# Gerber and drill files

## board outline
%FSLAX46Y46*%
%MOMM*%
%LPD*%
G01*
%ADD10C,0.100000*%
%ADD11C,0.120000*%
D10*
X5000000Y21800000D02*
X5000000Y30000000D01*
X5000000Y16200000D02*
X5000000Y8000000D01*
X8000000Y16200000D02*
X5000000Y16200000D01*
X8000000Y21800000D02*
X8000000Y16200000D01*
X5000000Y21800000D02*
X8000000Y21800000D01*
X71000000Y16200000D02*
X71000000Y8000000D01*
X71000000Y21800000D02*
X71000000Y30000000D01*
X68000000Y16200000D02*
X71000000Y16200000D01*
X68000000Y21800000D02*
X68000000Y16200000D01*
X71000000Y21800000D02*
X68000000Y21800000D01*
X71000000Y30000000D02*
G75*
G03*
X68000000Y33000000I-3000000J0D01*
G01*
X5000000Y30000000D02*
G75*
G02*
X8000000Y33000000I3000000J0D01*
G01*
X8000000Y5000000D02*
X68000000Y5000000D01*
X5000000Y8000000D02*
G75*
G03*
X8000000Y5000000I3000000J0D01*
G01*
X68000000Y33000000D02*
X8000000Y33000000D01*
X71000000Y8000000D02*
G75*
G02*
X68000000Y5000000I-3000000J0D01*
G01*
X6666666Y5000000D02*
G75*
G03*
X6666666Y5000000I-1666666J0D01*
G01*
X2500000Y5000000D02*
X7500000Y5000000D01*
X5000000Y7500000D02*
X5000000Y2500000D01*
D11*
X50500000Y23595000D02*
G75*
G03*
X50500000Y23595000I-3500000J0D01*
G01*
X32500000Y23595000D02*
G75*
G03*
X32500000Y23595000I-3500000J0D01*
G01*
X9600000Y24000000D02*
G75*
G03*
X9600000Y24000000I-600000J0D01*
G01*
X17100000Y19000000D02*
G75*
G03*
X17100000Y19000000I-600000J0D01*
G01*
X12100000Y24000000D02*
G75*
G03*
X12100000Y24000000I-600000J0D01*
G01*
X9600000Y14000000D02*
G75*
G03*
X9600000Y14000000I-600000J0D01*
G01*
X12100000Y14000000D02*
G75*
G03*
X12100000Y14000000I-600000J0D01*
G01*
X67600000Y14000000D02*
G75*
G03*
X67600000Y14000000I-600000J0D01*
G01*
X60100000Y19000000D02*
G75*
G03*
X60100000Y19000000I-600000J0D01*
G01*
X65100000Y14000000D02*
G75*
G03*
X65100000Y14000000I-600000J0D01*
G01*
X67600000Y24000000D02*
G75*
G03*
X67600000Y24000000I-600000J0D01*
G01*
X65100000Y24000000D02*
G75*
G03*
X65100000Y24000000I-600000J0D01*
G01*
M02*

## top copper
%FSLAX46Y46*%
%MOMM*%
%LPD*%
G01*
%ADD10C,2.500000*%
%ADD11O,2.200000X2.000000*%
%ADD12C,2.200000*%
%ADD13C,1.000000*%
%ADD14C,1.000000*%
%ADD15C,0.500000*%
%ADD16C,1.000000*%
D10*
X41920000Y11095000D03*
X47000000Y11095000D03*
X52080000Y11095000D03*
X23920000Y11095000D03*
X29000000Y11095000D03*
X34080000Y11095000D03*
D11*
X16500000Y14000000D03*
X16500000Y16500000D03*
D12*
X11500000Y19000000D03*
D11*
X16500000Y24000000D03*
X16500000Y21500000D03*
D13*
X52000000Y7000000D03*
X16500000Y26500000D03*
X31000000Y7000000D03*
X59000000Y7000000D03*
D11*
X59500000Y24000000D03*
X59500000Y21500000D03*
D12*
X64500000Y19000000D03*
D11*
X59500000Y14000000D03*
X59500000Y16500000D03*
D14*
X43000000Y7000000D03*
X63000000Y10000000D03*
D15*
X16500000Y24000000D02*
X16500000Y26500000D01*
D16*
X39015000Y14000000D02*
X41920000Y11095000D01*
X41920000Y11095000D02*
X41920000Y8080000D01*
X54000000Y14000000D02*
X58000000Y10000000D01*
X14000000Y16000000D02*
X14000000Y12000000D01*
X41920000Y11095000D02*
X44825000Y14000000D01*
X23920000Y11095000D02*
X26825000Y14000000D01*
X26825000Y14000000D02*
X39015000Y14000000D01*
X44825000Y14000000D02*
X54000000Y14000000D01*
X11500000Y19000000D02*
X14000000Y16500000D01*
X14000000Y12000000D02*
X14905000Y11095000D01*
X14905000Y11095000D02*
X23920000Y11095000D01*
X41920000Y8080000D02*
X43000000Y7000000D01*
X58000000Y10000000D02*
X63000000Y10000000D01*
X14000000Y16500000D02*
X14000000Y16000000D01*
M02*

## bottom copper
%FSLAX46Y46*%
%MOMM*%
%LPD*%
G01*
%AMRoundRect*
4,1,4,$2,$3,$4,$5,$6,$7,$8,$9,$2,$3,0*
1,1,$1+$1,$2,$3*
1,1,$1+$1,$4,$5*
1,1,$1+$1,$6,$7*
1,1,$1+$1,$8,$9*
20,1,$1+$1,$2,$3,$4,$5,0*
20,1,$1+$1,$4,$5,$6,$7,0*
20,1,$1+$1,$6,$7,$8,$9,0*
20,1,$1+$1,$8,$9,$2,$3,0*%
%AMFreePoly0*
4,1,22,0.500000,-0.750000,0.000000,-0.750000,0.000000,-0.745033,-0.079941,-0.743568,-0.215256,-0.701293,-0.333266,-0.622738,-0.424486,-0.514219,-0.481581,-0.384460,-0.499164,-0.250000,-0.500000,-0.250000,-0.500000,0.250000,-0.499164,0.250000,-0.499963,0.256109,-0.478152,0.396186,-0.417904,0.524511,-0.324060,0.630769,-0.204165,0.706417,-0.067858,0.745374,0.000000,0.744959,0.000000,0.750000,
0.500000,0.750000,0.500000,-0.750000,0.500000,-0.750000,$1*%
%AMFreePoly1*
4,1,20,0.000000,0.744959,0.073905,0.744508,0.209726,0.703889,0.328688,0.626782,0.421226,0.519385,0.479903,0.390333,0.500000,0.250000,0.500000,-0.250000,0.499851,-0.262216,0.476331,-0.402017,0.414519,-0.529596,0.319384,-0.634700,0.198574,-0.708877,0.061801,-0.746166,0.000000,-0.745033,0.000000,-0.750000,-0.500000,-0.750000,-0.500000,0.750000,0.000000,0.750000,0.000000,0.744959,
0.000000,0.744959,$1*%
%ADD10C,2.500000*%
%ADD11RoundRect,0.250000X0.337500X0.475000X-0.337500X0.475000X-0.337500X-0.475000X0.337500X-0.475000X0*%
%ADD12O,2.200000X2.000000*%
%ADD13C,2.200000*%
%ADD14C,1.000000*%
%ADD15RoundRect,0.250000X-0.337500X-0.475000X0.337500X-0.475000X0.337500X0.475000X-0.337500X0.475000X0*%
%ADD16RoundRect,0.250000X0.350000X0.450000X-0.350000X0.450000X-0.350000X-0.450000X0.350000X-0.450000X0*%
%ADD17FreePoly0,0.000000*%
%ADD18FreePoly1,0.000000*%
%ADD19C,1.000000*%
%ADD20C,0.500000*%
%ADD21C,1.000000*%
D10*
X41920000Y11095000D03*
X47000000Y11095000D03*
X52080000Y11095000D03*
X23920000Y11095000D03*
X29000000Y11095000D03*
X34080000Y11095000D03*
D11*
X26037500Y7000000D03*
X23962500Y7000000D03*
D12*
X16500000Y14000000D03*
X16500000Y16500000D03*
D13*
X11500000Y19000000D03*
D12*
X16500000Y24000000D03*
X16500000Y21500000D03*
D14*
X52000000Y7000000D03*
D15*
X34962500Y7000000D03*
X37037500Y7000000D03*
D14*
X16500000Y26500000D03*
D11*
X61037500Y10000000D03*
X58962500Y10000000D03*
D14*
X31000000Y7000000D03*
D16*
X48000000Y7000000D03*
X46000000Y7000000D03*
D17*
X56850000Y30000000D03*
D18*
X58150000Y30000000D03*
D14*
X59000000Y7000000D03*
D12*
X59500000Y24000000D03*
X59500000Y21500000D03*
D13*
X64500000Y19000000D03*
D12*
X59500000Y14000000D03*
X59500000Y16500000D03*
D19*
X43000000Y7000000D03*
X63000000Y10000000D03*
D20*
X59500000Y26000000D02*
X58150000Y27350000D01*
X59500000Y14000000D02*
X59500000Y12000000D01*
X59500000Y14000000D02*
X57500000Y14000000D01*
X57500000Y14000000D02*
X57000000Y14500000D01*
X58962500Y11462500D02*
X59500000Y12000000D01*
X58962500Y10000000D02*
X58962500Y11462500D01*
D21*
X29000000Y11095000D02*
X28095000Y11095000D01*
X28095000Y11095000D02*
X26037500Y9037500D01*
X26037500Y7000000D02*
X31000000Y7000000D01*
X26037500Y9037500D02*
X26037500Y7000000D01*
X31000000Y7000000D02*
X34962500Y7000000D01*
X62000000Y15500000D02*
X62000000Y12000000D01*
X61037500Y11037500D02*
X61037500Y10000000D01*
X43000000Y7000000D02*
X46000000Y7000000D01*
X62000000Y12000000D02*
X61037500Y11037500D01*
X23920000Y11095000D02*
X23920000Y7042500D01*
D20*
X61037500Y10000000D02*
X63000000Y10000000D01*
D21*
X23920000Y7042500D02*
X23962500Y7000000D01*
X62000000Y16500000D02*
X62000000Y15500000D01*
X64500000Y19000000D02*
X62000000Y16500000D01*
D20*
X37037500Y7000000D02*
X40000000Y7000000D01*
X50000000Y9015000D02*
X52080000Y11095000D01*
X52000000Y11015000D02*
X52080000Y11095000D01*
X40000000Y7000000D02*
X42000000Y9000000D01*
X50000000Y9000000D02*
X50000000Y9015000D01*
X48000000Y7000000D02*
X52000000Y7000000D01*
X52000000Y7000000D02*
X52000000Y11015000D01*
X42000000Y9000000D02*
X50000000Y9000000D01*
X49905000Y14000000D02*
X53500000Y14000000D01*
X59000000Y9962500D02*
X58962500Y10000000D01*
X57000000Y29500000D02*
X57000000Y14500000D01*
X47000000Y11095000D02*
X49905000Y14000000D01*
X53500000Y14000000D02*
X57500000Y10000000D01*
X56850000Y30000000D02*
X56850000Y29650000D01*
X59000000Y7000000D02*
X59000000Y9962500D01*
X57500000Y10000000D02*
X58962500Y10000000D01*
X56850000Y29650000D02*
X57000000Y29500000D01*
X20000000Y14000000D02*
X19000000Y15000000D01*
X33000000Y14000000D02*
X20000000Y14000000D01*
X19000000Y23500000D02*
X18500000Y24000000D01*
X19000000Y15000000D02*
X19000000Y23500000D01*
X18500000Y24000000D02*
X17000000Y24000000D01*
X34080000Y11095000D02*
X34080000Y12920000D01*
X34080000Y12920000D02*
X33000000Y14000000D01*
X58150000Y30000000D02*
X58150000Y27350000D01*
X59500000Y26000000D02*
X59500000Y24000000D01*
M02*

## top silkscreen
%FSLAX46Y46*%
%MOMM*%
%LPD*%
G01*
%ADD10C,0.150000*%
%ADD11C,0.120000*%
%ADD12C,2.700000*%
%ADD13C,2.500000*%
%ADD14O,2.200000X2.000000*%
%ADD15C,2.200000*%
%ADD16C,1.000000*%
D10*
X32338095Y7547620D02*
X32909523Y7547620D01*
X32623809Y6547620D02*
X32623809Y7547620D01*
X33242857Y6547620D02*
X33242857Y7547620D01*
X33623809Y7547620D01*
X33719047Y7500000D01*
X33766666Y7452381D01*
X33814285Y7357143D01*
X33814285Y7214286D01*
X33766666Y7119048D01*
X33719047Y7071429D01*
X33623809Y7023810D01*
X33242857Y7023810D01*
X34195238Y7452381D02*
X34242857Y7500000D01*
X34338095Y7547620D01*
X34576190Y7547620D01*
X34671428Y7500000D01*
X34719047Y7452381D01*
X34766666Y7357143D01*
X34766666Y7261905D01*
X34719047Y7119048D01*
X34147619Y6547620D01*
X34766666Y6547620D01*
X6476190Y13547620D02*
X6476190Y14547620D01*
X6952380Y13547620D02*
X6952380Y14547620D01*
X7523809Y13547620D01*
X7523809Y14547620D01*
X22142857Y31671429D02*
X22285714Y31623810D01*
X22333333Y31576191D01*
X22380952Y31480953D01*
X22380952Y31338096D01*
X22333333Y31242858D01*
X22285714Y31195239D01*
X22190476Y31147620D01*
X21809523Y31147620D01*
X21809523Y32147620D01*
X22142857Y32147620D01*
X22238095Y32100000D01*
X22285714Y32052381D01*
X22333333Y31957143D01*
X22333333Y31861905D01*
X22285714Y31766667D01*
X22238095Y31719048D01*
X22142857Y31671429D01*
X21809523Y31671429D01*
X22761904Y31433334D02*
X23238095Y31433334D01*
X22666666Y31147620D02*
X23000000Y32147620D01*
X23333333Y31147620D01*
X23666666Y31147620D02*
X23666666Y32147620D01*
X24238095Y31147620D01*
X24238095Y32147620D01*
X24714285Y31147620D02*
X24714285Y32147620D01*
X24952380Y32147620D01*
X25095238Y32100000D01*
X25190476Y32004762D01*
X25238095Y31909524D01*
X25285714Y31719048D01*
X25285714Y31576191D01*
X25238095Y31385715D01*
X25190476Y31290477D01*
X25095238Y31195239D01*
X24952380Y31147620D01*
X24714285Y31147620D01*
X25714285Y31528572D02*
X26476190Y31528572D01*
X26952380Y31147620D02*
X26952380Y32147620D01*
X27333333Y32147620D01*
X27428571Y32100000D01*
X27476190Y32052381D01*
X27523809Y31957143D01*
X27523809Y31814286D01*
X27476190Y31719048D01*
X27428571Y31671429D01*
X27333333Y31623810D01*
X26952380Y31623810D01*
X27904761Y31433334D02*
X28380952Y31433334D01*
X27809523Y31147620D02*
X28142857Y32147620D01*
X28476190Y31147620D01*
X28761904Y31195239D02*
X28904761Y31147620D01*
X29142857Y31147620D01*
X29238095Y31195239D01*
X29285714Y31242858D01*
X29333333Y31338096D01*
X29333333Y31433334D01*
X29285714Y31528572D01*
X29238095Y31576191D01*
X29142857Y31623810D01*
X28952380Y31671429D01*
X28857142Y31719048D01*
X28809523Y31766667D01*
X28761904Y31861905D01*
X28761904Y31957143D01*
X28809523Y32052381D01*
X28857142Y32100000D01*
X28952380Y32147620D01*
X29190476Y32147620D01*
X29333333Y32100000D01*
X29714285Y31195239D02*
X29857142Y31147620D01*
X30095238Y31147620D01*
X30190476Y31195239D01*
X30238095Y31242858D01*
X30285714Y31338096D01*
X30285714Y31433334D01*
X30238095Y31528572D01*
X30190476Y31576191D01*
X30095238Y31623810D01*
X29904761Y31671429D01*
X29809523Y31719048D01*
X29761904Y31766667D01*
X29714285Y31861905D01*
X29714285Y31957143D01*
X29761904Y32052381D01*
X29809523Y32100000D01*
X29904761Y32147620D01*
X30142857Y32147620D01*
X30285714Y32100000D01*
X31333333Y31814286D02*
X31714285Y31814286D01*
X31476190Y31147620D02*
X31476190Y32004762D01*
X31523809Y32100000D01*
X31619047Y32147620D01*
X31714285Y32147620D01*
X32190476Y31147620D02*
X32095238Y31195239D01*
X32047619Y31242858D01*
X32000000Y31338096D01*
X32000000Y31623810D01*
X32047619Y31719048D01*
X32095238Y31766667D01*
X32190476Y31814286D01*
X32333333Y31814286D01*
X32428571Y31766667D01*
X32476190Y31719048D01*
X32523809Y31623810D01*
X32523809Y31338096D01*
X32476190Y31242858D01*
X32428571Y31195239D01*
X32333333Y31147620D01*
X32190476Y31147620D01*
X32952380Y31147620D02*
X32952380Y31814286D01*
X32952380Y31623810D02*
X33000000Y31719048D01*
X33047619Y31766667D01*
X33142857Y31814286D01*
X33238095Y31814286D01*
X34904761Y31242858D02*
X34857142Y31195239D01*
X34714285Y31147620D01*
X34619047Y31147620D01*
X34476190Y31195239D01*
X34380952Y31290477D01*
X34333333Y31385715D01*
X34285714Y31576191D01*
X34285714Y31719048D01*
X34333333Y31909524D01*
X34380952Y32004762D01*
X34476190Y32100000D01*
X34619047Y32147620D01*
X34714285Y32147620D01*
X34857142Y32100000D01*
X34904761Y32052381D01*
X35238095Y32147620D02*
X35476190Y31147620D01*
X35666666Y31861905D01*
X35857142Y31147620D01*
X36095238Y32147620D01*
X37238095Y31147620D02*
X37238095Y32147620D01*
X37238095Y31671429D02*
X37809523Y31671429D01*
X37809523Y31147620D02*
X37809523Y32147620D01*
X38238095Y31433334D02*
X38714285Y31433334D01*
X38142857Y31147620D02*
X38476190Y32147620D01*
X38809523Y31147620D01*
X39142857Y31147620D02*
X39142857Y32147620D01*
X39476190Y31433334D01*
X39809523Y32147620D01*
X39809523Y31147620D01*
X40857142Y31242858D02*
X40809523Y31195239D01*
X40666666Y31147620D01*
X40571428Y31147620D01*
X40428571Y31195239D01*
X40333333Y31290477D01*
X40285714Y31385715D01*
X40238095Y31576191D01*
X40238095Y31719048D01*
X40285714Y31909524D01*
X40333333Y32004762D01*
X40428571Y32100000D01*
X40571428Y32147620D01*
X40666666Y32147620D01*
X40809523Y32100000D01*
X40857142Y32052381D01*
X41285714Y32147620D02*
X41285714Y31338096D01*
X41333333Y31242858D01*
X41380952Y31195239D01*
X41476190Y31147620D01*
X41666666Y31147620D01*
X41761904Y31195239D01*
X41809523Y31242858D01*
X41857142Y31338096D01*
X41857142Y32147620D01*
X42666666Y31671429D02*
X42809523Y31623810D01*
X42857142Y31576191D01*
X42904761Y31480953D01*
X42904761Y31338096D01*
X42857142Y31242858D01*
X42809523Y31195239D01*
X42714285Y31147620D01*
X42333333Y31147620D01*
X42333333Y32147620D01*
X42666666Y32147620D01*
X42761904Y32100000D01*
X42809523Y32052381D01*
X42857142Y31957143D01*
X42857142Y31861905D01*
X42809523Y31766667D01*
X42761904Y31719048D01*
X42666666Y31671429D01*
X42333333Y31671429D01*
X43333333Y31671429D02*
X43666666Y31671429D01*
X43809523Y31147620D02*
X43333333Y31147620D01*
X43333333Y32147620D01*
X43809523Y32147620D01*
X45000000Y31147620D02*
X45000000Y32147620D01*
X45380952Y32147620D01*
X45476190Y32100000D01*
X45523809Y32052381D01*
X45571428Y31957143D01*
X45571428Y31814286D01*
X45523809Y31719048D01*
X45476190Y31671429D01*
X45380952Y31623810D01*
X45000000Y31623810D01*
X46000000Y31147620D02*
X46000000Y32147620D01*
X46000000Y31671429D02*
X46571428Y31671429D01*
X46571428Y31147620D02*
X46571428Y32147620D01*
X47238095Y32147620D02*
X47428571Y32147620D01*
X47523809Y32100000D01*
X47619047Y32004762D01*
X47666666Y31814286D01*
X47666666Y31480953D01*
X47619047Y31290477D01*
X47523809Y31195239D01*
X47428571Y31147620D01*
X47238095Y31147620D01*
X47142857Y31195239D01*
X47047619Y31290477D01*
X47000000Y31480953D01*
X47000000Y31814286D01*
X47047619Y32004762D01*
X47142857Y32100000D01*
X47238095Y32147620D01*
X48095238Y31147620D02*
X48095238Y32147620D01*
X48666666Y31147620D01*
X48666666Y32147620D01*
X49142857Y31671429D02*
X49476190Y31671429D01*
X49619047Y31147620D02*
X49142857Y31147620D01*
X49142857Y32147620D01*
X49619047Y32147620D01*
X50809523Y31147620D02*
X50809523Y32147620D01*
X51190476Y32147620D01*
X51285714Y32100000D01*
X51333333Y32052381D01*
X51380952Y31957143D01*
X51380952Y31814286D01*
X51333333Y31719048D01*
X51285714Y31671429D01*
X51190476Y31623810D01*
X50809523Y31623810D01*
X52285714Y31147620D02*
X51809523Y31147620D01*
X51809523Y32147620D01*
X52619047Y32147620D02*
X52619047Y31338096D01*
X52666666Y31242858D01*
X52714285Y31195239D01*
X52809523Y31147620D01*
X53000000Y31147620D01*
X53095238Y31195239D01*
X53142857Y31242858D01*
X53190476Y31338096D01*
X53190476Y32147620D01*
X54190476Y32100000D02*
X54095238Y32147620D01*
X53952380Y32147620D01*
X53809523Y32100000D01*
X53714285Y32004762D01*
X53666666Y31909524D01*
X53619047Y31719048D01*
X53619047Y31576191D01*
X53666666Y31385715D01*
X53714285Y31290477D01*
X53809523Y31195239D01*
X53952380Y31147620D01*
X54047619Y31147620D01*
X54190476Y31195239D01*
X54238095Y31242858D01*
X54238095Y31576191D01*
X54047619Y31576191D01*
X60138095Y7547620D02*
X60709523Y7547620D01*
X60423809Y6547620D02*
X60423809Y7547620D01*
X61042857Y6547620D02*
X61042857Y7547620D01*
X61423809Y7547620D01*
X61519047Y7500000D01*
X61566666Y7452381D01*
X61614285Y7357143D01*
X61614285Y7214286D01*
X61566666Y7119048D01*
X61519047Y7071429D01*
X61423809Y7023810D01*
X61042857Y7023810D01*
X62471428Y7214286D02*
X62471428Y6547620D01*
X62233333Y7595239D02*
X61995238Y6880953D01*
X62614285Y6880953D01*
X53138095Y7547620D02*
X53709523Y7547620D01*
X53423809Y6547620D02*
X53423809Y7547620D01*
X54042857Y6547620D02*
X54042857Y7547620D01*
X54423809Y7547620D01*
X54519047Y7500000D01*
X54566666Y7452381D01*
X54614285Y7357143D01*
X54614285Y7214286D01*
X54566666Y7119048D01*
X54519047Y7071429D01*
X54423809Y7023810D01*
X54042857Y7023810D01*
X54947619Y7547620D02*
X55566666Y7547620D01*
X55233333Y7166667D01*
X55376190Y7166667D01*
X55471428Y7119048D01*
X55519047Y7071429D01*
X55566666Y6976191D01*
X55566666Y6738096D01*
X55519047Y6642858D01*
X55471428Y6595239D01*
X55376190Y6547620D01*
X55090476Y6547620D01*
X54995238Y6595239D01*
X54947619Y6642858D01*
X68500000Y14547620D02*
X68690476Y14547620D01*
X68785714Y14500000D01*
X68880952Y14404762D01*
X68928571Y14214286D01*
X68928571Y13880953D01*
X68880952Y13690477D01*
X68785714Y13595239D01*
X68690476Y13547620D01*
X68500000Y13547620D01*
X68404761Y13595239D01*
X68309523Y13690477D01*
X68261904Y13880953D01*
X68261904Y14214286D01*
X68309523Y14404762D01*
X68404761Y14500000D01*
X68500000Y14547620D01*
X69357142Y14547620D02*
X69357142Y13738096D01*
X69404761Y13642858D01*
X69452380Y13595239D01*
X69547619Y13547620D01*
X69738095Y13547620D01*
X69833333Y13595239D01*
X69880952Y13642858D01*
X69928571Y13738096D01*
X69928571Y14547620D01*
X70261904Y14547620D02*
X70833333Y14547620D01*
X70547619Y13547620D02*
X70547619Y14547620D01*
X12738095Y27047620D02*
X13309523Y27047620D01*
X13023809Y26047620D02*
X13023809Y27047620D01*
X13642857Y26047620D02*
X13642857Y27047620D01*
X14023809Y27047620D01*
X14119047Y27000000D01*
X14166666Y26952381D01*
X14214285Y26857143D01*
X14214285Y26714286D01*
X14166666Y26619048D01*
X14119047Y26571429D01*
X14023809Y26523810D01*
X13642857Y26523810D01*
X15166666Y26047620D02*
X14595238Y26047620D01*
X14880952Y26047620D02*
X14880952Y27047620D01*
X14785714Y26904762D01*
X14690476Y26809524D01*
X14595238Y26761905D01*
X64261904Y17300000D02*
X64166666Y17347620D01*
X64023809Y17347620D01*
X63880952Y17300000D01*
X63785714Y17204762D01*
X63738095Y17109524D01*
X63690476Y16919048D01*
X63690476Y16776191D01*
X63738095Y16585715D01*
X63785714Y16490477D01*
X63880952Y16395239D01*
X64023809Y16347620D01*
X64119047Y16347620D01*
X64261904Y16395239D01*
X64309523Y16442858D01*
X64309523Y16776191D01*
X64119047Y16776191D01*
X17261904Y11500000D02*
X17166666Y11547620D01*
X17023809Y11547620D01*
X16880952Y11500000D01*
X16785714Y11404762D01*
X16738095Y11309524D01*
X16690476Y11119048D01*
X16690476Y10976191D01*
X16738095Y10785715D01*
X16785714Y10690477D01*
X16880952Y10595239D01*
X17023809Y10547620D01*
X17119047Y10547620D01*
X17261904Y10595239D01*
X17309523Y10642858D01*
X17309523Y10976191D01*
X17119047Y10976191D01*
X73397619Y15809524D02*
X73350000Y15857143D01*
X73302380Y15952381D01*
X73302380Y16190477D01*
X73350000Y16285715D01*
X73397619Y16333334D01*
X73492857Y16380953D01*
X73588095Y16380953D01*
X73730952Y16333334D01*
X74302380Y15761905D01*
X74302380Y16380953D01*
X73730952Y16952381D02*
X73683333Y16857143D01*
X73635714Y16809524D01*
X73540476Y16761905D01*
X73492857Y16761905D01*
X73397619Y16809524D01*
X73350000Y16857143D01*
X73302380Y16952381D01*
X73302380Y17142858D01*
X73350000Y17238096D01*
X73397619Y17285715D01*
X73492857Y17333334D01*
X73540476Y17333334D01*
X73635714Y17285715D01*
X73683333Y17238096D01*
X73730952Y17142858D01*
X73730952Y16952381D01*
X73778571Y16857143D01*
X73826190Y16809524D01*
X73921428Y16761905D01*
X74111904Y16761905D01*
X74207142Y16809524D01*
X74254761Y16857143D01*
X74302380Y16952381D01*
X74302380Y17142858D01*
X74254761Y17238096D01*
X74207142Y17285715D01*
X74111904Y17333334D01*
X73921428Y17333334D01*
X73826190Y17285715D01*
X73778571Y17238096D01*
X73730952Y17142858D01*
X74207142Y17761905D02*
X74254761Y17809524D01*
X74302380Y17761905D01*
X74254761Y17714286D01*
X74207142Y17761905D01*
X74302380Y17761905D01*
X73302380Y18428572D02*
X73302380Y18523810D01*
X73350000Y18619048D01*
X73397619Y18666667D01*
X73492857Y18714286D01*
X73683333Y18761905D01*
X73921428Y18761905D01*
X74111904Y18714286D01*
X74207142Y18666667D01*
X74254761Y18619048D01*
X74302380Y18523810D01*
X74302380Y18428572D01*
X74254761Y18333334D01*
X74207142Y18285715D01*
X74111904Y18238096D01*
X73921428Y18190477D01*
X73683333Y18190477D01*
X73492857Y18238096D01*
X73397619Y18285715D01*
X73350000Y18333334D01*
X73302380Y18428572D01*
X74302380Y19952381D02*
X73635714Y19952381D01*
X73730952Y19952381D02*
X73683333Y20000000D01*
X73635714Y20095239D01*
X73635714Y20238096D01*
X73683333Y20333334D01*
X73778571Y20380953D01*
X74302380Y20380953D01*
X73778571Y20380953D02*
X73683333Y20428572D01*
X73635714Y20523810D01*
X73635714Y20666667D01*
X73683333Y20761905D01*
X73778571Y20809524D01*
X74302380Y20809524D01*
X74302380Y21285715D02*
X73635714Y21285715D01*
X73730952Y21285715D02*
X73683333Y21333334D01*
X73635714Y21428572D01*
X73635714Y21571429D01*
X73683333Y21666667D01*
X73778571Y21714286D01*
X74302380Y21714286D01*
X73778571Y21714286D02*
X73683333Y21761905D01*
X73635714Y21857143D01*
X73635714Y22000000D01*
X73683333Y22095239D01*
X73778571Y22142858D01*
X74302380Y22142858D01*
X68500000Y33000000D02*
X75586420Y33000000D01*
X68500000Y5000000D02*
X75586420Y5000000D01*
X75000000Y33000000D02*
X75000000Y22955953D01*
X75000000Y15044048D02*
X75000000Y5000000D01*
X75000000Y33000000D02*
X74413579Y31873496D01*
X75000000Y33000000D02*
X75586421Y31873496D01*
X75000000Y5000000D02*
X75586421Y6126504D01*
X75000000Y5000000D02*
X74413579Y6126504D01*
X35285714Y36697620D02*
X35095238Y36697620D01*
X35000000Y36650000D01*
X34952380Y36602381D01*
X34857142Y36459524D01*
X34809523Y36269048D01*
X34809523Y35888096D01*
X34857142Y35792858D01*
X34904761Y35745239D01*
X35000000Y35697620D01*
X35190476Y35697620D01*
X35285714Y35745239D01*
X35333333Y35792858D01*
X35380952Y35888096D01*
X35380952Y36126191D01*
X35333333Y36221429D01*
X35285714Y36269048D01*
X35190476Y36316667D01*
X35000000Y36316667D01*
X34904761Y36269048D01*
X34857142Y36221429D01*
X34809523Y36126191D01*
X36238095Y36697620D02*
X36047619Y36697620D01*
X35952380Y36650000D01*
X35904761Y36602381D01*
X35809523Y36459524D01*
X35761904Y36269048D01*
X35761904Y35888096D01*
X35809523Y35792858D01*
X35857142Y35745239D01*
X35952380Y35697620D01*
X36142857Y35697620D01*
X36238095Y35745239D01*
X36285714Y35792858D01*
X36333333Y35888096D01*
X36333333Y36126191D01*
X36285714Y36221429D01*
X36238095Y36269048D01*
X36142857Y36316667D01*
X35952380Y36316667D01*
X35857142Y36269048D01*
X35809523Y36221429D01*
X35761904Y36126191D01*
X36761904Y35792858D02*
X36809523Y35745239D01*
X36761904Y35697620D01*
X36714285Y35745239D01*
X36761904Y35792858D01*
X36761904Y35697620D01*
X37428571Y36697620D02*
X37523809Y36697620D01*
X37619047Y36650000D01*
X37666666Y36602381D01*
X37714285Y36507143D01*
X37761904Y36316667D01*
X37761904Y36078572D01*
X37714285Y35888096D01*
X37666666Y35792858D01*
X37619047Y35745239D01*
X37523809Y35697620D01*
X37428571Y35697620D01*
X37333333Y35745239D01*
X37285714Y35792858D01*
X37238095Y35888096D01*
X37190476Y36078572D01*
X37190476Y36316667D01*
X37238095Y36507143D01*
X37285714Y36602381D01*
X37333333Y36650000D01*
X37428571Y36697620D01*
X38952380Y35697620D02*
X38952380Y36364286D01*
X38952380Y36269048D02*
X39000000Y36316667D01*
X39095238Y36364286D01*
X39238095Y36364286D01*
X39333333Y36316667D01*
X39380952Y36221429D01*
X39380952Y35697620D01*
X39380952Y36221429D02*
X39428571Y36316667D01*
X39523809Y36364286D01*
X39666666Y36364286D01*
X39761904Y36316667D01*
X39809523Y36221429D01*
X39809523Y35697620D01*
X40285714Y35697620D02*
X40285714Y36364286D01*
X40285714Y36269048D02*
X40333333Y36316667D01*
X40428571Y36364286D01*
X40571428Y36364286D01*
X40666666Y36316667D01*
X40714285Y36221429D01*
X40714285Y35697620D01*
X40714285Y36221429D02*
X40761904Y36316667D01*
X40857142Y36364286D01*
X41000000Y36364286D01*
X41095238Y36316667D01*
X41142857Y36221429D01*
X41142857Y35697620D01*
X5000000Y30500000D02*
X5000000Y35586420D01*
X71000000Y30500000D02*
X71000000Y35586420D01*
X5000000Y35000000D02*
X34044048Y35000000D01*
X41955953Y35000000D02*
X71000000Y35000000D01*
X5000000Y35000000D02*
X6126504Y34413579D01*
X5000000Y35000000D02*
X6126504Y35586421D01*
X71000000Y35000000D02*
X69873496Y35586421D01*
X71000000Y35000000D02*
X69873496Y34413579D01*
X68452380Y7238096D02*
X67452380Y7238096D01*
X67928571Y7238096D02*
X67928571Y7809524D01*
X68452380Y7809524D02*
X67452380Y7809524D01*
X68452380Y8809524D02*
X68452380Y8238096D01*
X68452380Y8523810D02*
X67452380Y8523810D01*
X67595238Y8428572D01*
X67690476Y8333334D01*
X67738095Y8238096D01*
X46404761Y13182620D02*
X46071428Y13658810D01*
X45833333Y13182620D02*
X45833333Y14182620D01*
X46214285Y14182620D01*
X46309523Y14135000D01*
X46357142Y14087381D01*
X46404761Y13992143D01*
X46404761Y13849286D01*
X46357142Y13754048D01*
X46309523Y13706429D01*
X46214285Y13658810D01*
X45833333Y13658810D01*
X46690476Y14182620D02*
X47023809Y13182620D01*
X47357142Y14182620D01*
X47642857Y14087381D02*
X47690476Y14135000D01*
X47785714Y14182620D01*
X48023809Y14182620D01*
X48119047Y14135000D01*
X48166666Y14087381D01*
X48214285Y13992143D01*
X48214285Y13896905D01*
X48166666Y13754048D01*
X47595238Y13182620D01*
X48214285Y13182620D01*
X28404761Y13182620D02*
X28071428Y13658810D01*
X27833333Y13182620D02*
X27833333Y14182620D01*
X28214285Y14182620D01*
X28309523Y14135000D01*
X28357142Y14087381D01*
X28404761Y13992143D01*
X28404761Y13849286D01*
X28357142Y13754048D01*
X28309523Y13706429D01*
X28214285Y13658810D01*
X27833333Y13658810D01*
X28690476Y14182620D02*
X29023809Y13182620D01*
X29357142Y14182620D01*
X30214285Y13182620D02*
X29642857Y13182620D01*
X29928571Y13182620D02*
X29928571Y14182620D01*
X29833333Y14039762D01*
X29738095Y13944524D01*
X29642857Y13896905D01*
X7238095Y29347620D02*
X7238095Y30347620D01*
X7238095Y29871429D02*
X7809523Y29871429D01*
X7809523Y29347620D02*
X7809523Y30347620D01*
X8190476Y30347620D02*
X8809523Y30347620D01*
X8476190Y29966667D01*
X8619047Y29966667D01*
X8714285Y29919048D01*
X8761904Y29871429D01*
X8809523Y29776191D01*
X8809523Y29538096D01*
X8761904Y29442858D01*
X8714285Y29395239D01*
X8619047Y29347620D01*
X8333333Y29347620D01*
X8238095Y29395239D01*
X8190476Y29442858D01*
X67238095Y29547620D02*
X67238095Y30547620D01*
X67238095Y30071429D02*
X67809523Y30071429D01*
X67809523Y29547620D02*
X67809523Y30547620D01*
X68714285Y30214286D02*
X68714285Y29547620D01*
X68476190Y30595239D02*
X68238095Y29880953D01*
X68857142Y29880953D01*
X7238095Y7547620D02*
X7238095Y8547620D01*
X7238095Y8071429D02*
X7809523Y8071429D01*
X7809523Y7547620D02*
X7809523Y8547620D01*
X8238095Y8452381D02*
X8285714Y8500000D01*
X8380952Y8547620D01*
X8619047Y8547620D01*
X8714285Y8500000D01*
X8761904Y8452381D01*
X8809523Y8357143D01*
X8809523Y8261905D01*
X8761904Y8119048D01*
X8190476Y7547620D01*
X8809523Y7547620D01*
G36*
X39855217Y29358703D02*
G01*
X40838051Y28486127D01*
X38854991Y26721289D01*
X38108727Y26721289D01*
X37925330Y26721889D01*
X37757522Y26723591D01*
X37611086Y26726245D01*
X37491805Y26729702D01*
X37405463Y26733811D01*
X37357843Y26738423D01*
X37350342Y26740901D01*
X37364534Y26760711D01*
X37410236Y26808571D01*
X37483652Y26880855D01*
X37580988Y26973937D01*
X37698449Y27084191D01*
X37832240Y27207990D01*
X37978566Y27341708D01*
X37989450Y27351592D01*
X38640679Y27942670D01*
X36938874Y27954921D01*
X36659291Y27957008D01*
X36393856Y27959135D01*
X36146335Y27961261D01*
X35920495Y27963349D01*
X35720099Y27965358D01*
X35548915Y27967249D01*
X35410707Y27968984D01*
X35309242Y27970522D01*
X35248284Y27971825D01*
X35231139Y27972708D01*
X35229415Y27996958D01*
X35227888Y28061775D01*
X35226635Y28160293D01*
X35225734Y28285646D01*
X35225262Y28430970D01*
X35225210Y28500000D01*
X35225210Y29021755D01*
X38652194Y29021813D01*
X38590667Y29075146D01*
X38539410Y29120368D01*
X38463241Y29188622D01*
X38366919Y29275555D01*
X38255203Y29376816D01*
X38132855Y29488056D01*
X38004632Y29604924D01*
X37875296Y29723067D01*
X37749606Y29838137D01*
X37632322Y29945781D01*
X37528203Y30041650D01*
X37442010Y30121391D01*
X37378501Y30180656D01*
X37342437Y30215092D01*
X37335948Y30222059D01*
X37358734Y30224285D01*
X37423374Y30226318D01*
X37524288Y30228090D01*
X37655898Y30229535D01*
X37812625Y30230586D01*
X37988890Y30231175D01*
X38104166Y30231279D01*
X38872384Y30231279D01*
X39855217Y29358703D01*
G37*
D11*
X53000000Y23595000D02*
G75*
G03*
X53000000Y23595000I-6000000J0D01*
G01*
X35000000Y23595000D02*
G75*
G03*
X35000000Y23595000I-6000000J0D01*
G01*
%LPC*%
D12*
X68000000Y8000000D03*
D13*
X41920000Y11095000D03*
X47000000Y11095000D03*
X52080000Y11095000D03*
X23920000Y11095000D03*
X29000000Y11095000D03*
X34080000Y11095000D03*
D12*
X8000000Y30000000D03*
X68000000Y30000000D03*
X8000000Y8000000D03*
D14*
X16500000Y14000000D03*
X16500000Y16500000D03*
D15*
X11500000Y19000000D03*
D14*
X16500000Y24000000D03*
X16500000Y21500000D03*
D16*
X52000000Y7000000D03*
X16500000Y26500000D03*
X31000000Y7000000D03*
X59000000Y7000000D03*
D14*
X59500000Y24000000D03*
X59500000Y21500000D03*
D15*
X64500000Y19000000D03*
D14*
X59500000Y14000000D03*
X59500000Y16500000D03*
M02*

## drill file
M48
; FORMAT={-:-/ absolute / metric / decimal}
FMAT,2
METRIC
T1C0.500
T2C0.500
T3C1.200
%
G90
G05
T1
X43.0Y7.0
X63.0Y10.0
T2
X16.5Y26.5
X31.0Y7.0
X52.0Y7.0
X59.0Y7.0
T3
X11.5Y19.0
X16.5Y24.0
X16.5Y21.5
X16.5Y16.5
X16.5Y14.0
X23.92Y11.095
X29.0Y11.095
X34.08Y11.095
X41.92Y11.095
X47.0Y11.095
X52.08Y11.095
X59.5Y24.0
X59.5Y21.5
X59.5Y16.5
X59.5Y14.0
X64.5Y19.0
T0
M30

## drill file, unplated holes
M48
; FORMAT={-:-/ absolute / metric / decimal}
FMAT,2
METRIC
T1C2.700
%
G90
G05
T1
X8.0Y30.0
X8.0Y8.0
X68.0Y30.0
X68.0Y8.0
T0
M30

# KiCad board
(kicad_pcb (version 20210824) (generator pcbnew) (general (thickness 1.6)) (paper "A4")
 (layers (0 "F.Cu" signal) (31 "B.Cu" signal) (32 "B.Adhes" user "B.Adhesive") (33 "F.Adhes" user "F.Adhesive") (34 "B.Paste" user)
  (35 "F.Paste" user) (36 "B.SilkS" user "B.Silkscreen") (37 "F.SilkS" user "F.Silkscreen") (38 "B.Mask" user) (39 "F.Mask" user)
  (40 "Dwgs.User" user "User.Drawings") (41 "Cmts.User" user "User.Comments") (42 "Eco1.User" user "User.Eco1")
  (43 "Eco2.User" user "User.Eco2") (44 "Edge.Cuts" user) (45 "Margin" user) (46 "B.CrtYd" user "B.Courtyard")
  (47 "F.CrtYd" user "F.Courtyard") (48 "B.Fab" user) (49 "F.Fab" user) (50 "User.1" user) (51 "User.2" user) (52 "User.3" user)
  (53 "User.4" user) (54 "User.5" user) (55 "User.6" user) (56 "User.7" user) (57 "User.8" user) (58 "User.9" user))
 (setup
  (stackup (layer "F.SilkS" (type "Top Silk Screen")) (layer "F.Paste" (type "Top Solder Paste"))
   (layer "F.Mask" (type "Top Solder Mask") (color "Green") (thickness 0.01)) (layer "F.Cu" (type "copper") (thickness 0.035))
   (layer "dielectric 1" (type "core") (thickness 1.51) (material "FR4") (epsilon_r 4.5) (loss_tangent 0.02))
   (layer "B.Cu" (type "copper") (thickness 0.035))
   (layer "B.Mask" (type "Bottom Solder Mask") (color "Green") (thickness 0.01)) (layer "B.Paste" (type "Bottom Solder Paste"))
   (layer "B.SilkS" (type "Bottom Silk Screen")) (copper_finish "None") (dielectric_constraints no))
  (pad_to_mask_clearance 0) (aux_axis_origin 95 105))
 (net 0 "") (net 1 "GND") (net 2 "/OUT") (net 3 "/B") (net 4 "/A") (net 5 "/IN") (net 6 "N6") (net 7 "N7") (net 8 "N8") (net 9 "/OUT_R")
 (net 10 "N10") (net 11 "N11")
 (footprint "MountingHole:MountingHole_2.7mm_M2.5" (layer "F.Cu") (at 163 97)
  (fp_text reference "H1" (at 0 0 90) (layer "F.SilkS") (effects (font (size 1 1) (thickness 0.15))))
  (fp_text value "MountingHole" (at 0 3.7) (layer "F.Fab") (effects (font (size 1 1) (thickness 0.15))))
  (pad "" np_thru_hole circle locked (at 0 0) (size 2.7 2.7) (drill 2.7) (layers *.Cu *.Mask)))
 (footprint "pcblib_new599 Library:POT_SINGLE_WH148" (layer "F.Cu") (at 142 93.905)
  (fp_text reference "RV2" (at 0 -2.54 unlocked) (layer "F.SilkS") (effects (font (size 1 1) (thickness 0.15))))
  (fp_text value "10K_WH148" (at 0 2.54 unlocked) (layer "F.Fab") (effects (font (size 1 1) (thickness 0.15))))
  (fp_circle (center 0 -12.5) (end 6 -12.5) (layer "F.SilkS") (width 0.12) (fill none))
  (fp_circle (center 0 -12.5) (end 3.5 -12.5) (layer "Edge.Cuts") (width 0.12) (fill none))
  (pad "1" thru_hole circle (at -5.08 0) (size 2.5 2.5) (drill 1.2) (layers *.Cu *.Mask) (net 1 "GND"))
  (pad "2" thru_hole circle (at 0 0) (size 2.5 2.5) (drill 1.2) (layers *.Cu *.Mask) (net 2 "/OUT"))
  (pad "3" thru_hole circle (at 5.08 0) (size 2.5 2.5) (drill 1.2) (layers *.Cu *.Mask) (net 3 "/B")))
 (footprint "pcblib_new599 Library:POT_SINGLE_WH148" (layer "F.Cu") (at 124 93.905)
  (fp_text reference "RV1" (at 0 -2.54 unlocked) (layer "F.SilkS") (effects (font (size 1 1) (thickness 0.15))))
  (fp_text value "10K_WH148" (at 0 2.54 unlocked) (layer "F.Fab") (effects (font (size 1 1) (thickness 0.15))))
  (fp_circle (center 0 -12.5) (end 6 -12.5) (layer "F.SilkS") (width 0.12) (fill none))
  (fp_circle (center 0 -12.5) (end 3.5 -12.5) (layer "Edge.Cuts") (width 0.12) (fill none))
  (pad "1" thru_hole circle (at -5.08 0) (size 2.5 2.5) (drill 1.2) (layers *.Cu *.Mask) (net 1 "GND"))
  (pad "2" thru_hole circle (at 0 0) (size 2.5 2.5) (drill 1.2) (layers *.Cu *.Mask) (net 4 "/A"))
  (pad "3" thru_hole circle (at 5.08 0) (size 2.5 2.5) (drill 1.2) (layers *.Cu *.Mask) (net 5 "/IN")))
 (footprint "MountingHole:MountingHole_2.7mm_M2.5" (layer "F.Cu") (at 103 75)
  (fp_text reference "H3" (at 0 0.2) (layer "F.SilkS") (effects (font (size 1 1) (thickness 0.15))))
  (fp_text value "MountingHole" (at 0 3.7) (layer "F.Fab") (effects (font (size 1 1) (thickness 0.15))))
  (pad "" np_thru_hole circle locked (at 0 0) (size 2.7 2.7) (drill 2.7) (layers *.Cu *.Mask)))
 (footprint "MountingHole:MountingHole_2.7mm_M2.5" (layer "F.Cu") (at 163 75)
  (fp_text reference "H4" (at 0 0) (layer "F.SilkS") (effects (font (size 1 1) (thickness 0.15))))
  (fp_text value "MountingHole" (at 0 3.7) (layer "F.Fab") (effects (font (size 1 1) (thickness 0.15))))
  (pad "" np_thru_hole circle locked (at 0 0) (size 2.7 2.7) (drill 2.7) (layers *.Cu *.Mask)))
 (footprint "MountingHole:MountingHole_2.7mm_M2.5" (layer "F.Cu") (at 103 97)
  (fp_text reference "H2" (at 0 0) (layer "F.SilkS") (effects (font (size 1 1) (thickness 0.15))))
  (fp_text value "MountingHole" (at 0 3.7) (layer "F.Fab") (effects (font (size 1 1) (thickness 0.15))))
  (pad "" np_thru_hole circle locked (at 0 0) (size 2.7 2.7) (drill 2.7) (layers *.Cu *.Mask)))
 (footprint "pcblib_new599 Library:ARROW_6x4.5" (layer "F.Cu") (at 133 76.5 180)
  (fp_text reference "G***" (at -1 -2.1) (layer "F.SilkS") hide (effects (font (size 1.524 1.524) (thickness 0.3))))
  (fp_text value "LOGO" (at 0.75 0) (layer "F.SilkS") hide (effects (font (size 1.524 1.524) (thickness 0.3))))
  (fp_poly
   (pts (xy 0.07467 -1.778111) (xy 0.242478 -1.776409) (xy 0.388914 -1.773755) (xy 0.508195 -1.770298) (xy 0.594537 -1.766189)
    (xy 0.642157 -1.761577) (xy 0.649658 -1.759099) (xy 0.635466 -1.739289) (xy 0.589764 -1.691429) (xy 0.516348 -1.619145)
    (xy 0.419012 -1.526063) (xy 0.301551 -1.415809) (xy 0.16776 -1.29201) (xy 0.021434 -1.158292) (xy 0.01055 -1.148408)
    (xy -0.640679 -0.55733) (xy 1.061126 -0.545079) (xy 1.340709 -0.542992) (xy 1.606144 -0.540865) (xy 1.853665 -0.538739)
    (xy 2.079505 -0.536651) (xy 2.279901 -0.534642) (xy 2.451085 -0.532751) (xy 2.589293 -0.531016) (xy 2.690758 -0.529478)
    (xy 2.751716 -0.528175) (xy 2.768861 -0.527292) (xy 2.770585 -0.503042) (xy 2.772112 -0.438225) (xy 2.773365 -0.339707)
    (xy 2.774266 -0.214354) (xy 2.774738 -0.06903) (xy 2.77479 0) (xy 2.77479 0.521755) (xy -0.652194 0.521813) (xy -0.590667 0.575146)
    (xy -0.53941 0.620368) (xy -0.463241 0.688622) (xy -0.366919 0.775555) (xy -0.255203 0.876816) (xy -0.132855 0.988056)
    (xy -0.004632 1.104924) (xy 0.124704 1.223067) (xy 0.250394 1.338137) (xy 0.367678 1.445781) (xy 0.471797 1.54165) (xy 0.55799 1.621391)
    (xy 0.621499 1.680656) (xy 0.657563 1.715092) (xy 0.664052 1.722059) (xy 0.641266 1.724285) (xy 0.576626 1.726318) (xy 0.475712 1.72809)
    (xy 0.344102 1.729535) (xy 0.187375 1.730586) (xy 0.01111 1.731175) (xy -0.104166 1.731279) (xy -0.872384 1.731279)
    (xy -1.855217 0.858703) (xy -2.838051 -0.013873) (xy -0.854991 -1.778711) (xy -0.108727 -1.778711))
   (layer "F.SilkS") (width 0) (fill solid)))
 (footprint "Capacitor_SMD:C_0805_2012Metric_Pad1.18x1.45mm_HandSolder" (layer "B.Cu") (at 120 98 180)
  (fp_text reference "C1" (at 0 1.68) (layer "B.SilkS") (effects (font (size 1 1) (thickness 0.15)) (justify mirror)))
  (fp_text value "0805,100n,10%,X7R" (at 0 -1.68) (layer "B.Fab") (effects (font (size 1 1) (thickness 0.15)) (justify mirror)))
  (pad "1" smd roundrect locked (at -1.0375 0 180) (size 1.175 1.45) (layers "B.Cu" "B.Paste" "B.Mask") (roundrect_rratio 0.212766)
   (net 4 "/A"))
  (pad "2" smd roundrect locked (at 1.0375 0 180) (size 1.175 1.45) (layers "B.Cu" "B.Paste" "B.Mask") (roundrect_rratio 0.212766)
   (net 1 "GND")))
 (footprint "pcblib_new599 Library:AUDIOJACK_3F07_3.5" (layer "B.Cu") (at 106.5 86 90)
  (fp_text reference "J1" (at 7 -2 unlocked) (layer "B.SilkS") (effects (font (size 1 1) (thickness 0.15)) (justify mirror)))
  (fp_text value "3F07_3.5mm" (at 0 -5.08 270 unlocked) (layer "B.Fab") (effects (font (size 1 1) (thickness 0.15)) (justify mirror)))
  (fp_circle (center -5 -2.5) (end -4.4 -2.5) (layer "Edge.Cuts") (width 0.12) (fill none))
  (fp_circle (center -5 0) (end -4.4 0) (layer "Edge.Cuts") (width 0.12) (fill none))
  (fp_circle (center 5 -2.5) (end 5.6 -2.5) (layer "Edge.Cuts") (width 0.12) (fill none))
  (fp_circle (center 5 0) (end 5.6 0) (layer "Edge.Cuts") (width 0.12) (fill none))
  (fp_circle (center 0 5) (end 0.6 5) (layer "Edge.Cuts") (width 0.12) (fill none))
  (pad "R" thru_hole oval (at -5 5 90) (size 2 2.2) (drill 1.2) (layers *.Cu *.Mask) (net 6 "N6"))
  (pad "RN" thru_hole oval (at -2.5 5 90) (size 2 2.2) (drill 1.2) (layers *.Cu *.Mask) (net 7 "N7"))
  (pad "S" thru_hole circle (at 0 0 90) (size 2.2 2.2) (drill 1.2) (layers *.Cu *.Mask) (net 1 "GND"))
  (pad "T" thru_hole oval (at 5 5 90) (size 2 2.2) (drill 1.2) (layers *.Cu *.Mask) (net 5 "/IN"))
  (pad "TN" thru_hole oval (at 2.5 5 90) (size 2 2.2) (drill 1.2) (layers *.Cu *.Mask) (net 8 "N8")))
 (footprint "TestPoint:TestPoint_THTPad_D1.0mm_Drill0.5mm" (layer "B.Cu") (at 147 98 180)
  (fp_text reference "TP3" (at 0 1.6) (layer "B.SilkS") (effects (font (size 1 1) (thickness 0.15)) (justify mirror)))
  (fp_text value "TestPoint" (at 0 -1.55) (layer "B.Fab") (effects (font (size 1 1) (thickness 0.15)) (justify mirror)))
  (pad "1" thru_hole circle locked (at 0 0 180) (size 1 1) (drill 0.5) (layers *.Cu *.Mask) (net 3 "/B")))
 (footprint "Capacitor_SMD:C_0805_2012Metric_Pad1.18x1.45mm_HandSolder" (layer "B.Cu") (at 131 98)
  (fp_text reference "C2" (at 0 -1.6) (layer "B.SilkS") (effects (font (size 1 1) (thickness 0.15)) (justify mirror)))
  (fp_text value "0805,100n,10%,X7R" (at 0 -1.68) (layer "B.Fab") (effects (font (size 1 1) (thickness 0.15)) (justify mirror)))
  (pad "1" smd roundrect locked (at -1.0375 0) (size 1.175 1.45) (layers "B.Cu" "B.Paste" "B.Mask") (roundrect_rratio 0.212766) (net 4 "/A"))
  (pad "2" smd roundrect locked (at 1.0375 0) (size 1.175 1.45) (layers "B.Cu" "B.Paste" "B.Mask") (roundrect_rratio 0.212766) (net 3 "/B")))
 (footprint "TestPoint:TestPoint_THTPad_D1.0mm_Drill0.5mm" (layer "B.Cu") (at 111.5 78.5 180)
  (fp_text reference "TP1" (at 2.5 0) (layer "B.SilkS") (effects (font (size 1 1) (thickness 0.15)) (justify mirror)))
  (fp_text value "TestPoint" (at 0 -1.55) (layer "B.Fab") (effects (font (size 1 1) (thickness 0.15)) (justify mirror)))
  (pad "1" thru_hole circle locked (at 0 0 180) (size 1 1) (drill 0.5) (layers *.Cu *.Mask) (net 5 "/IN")))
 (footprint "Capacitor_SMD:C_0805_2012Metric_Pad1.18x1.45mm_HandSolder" (layer "B.Cu") (at 155 95 180)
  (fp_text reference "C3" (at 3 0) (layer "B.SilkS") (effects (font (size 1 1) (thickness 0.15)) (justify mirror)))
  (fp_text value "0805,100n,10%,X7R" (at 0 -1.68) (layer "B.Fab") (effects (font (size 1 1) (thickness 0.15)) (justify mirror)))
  (pad "1" smd roundrect locked (at -1.0375 0 180) (size 1.175 1.45) (layers "B.Cu" "B.Paste" "B.Mask") (roundrect_rratio 0.212766)
   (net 1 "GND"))
  (pad "2" smd roundrect locked (at 1.0375 0 180) (size 1.175 1.45) (layers "B.Cu" "B.Paste" "B.Mask") (roundrect_rratio 0.212766)
   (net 2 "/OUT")))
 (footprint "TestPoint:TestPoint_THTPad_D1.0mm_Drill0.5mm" (layer "B.Cu") (at 126 98 180)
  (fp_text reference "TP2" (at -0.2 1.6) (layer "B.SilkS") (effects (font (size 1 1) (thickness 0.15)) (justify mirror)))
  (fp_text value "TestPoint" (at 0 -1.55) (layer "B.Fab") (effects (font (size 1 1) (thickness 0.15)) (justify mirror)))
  (pad "1" thru_hole circle locked (at 0 0 180) (size 1 1) (drill 0.5) (layers *.Cu *.Mask) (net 4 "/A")))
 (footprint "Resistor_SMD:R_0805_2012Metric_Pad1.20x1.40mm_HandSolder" (layer "B.Cu") (at 142 98 180)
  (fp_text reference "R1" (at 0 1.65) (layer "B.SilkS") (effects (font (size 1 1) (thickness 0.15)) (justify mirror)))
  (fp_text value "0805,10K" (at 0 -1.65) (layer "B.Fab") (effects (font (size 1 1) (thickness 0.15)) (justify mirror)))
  (pad "1" smd roundrect locked (at -1 0 180) (size 1.2 1.4) (layers "B.Cu" "B.Paste" "B.Mask") (roundrect_rratio 0.208333) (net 3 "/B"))
  (pad "2" smd roundrect locked (at 1 0 180) (size 1.2 1.4) (layers "B.Cu" "B.Paste" "B.Mask") (roundrect_rratio 0.208333) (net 1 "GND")))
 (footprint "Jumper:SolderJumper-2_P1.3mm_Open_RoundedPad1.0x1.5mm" (layer "B.Cu") (at 152.5 75)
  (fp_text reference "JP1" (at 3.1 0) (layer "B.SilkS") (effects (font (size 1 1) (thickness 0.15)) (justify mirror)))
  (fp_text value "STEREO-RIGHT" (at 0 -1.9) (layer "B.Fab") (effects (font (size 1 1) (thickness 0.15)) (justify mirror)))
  (pad "1" smd custom locked (at -0.65 0) (size 1 0.5) (layers "B.Cu" "B.Mask") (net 2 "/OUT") (zone_connect 2)
   (options (clearance outline) (anchor rect)) (primitives))
  (pad "2" smd custom locked (at 0.65 0) (size 1 0.5) (layers "B.Cu" "B.Mask") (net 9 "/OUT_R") (zone_connect 2)
   (options (clearance outline) (anchor rect)) (primitives)))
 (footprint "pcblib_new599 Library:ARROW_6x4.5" (layer "B.Cu") (at 113 75 180)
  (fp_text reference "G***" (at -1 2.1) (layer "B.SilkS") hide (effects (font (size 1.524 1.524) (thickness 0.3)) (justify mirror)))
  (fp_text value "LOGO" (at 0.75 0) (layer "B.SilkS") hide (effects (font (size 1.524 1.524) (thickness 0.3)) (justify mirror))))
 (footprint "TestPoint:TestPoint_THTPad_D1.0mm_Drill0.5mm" (layer "B.Cu") (at 154 98 180)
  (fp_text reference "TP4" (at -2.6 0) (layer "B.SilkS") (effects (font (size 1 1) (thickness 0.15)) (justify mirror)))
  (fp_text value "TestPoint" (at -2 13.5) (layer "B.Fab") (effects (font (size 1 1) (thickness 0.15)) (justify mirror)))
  (pad "1" thru_hole circle locked (at 0 0 180) (size 1 1) (drill 0.5) (layers *.Cu *.Mask) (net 2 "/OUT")))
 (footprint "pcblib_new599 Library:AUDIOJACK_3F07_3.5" (layer "B.Cu") (at 159.5 86 -90)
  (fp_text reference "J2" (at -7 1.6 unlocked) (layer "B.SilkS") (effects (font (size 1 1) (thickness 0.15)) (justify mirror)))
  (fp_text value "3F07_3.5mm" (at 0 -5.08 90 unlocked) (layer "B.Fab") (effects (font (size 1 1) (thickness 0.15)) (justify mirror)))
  (fp_circle (center 5 -2.5) (end 5.6 -2.5) (layer "Edge.Cuts") (width 0.12) (fill none))
  (fp_circle (center 5 0) (end 5.6 0) (layer "Edge.Cuts") (width 0.12) (fill none))
  (fp_circle (center -5 0) (end -4.4 0) (layer "Edge.Cuts") (width 0.12) (fill none))
  (fp_circle (center 0 5) (end 0.6 5) (layer "Edge.Cuts") (width 0.12) (fill none))
  (fp_circle (center -5 -2.5) (end -4.4 -2.5) (layer "Edge.Cuts") (width 0.12) (fill none))
  (pad "R" thru_hole oval (at -5 5 270) (size 2 2.2) (drill 1.2) (layers *.Cu *.Mask) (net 9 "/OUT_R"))
  (pad "RN" thru_hole oval (at -2.5 5 270) (size 2 2.2) (drill 1.2) (layers *.Cu *.Mask) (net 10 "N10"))
  (pad "S" thru_hole circle (at 0 0 270) (size 2.2 2.2) (drill 1.2) (layers *.Cu *.Mask) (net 1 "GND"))
  (pad "T" thru_hole oval (at 5 5 270) (size 2 2.2) (drill 1.2) (layers *.Cu *.Mask) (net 2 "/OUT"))
  (pad "TN" thru_hole oval (at 2.5 5 270) (size 2 2.2) (drill 1.2) (layers *.Cu *.Mask) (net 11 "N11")))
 (gr_arc (start 163 75) (end 163 72) (angle 90) (layer "Edge.Cuts") (width 0.1))
 (gr_line (start 100 83.2) (end 100 75) (layer "Edge.Cuts") (width 0.1))
 (gr_line (start 103 83.2) (end 103 88.8) (layer "Edge.Cuts") (width 0.1))
 (gr_line (start 166 83.2) (end 166 75) (layer "Edge.Cuts") (width 0.1))
 (gr_arc (start 103 75) (end 103 72) (angle -90) (layer "Edge.Cuts") (width 0.1))
 (gr_line (start 163 83.2) (end 163 88.8) (layer "Edge.Cuts") (width 0.1))
 (gr_line (start 163 88.8) (end 166 88.8) (layer "Edge.Cuts") (width 0.1))
 (gr_line (start 166 83.2) (end 163 83.2) (layer "Edge.Cuts") (width 0.1))
 (gr_line (start 103 100) (end 163 100) (layer "Edge.Cuts") (width 0.1))
 (gr_line (start 103 88.8) (end 100 88.8) (layer "Edge.Cuts") (width 0.1))
 (gr_line (start 100 88.8) (end 100 97) (layer "Edge.Cuts") (width 0.1))
 (gr_line (start 100 83.2) (end 103 83.2) (layer "Edge.Cuts") (width 0.1))
 (gr_arc (start 103 97) (end 103 100) (angle 90) (layer "Edge.Cuts") (width 0.1))
 (gr_line (start 163 72) (end 103 72) (layer "Edge.Cuts") (width 0.1))
 (gr_line (start 166 88.8) (end 166 97) (layer "Edge.Cuts") (width 0.1))
 (gr_arc (start 163 97) (end 163 100) (angle -90) (layer "Edge.Cuts") (width 0.1))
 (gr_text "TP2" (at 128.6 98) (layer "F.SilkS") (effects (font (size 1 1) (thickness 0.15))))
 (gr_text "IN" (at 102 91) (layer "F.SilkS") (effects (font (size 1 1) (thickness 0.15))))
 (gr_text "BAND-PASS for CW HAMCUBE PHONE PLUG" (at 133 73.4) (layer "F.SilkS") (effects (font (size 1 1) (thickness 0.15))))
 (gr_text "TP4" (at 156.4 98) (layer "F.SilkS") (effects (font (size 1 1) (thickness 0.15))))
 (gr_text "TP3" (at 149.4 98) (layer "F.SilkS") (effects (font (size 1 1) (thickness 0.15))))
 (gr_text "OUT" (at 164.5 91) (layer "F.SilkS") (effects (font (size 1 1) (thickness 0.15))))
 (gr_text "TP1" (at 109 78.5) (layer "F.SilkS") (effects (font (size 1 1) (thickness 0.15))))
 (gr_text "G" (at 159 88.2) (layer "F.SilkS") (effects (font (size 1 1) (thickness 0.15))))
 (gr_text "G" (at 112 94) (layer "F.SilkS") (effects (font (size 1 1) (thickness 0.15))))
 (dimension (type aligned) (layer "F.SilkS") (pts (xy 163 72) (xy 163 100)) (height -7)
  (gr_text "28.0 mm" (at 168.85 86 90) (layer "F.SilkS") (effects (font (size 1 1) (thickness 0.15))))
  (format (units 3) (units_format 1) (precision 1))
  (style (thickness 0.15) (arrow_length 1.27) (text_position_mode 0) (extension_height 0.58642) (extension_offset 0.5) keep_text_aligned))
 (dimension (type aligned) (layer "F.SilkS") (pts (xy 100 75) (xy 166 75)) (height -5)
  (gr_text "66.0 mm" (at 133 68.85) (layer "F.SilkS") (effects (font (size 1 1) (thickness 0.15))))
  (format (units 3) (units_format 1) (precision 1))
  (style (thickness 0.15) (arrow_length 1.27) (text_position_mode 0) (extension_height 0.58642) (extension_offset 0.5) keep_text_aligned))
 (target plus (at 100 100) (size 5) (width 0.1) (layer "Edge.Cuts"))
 (segment (start 124 93.905) (end 123.095 93.905) (width 1) (layer "B.Cu") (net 4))
 (segment (start 123.095 93.905) (end 121.0375 95.9625) (width 1) (layer "B.Cu") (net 4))
 (segment (start 121.0375 98) (end 126 98) (width 1) (layer "B.Cu") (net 4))
 (segment (start 121.0375 95.9625) (end 121.0375 98) (width 1) (layer "B.Cu") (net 4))
 (segment (start 126 98) (end 129.9625 98) (width 1) (layer "B.Cu") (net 4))
 (segment (start 134.015 91) (end 136.92 93.905) (width 1) (layer "F.Cu") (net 1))
 (segment (start 136.92 93.905) (end 136.92 96.92) (width 1) (layer "F.Cu") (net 1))
 (segment (start 149 91) (end 153 95) (width 1) (layer "F.Cu") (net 1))
 (segment (start 109 89) (end 109 93) (width 1) (layer "F.Cu") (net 1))
 (segment (start 136.92 93.905) (end 139.825 91) (width 1) (layer "F.Cu") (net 1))
 (segment (start 118.92 93.905) (end 121.825 91) (width 1) (layer "F.Cu") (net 1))
 (segment (start 121.825 91) (end 134.015 91) (width 1) (layer "F.Cu") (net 1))
 (segment (start 139.825 91) (end 149 91) (width 1) (layer "F.Cu") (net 1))
 (segment (start 106.5 86) (end 109 88.5) (width 1) (layer "F.Cu") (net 1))
 (segment (start 109 93) (end 109.905 93.905) (width 1) (layer "F.Cu") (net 1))
 (segment (start 109.905 93.905) (end 118.92 93.905) (width 1) (layer "F.Cu") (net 1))
 (segment (start 136.92 96.92) (end 138 98) (width 1) (layer "F.Cu") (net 1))
 (segment (start 153 95) (end 158 95) (width 1) (layer "F.Cu") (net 1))
 (segment (start 109 88.5) (end 109 89) (width 1) (layer "F.Cu") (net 1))
 (via (at 138 98) (size 1) (drill 0.5) (layers "F.Cu" "B.Cu") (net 1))
 (via (at 158 95) (size 1) (drill 0.5) (layers "F.Cu" "B.Cu") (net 1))
 (segment (start 157 89.5) (end 157 93) (width 1) (layer "B.Cu") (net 1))
 (segment (start 156.0375 93.9625) (end 156.0375 95) (width 1) (layer "B.Cu") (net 1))
 (segment (start 138 98) (end 141 98) (width 1) (layer "B.Cu") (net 1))
 (segment (start 157 93) (end 156.0375 93.9625) (width 1) (layer "B.Cu") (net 1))
 (segment (start 118.92 93.905) (end 118.92 97.9575) (width 1) (layer "B.Cu") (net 1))
 (segment (start 156.0375 95) (end 158 95) (width 0.5) (layer "B.Cu") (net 1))
 (segment (start 118.92 97.9575) (end 118.9625 98) (width 1) (layer "B.Cu") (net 1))
 (segment (start 157 88.5) (end 157 89.5) (width 1) (layer "B.Cu") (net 1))
 (segment (start 159.5 86) (end 157 88.5) (width 1) (layer "B.Cu") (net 1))
 (segment (start 132.0375 98) (end 135 98) (width 0.5) (layer "B.Cu") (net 3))
 (segment (start 145 95.985) (end 147.08 93.905) (width 0.5) (layer "B.Cu") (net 3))
 (segment (start 147 93.985) (end 147.08 93.905) (width 0.5) (layer "B.Cu") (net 3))
 (segment (start 135 98) (end 137 96) (width 0.5) (layer "B.Cu") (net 3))
 (segment (start 145 96) (end 145 95.985) (width 0.5) (layer "B.Cu") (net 3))
 (segment (start 143 98) (end 147 98) (width 0.5) (layer "B.Cu") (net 3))
 (segment (start 147 98) (end 147 93.985) (width 0.5) (layer "B.Cu") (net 3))
 (segment (start 137 96) (end 145 96) (width 0.5) (layer "B.Cu") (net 3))
 (segment (start 144.905 91) (end 148.5 91) (width 0.5) (layer "B.Cu") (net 2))
 (segment (start 154 95.0375) (end 153.9625 95) (width 0.5) (layer "B.Cu") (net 2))
 (segment (start 154.5 91) (end 154.5 93) (width 0.5) (layer "B.Cu") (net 2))
 (segment (start 152 75.5) (end 152 90.5) (width 0.5) (layer "B.Cu") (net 2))
 (segment (start 153.9625 93.5375) (end 154.5 93) (width 0.5) (layer "B.Cu") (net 2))
 (segment (start 142 93.905) (end 144.905 91) (width 0.5) (layer "B.Cu") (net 2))
 (segment (start 154.5 91) (end 152.5 91) (width 0.5) (layer "B.Cu") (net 2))
 (segment (start 148.5 91) (end 152.5 95) (width 0.5) (layer "B.Cu") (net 2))
 (segment (start 153.9625 95) (end 153.9625 93.5375) (width 0.5) (layer "B.Cu") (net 2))
 (segment (start 151.85 75) (end 151.85 75.35) (width 0.5) (layer "B.Cu") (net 2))
 (segment (start 154 98) (end 154 95.0375) (width 0.5) (layer "B.Cu") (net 2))
 (segment (start 152.5 95) (end 153.9625 95) (width 0.5) (layer "B.Cu") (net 2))
 (segment (start 151.85 75.35) (end 152 75.5) (width 0.5) (layer "B.Cu") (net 2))
 (segment (start 152.5 91) (end 152 90.5) (width 0.5) (layer "B.Cu") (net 2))
 (segment (start 111.5 81) (end 111.5 78.5) (width 0.5) (layer "F.Cu") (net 5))
 (segment (start 115 91) (end 114 90) (width 0.5) (layer "B.Cu") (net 5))
 (segment (start 128 91) (end 115 91) (width 0.5) (layer "B.Cu") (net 5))
 (segment (start 114 81.5) (end 113.5 81) (width 0.5) (layer "B.Cu") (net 5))
 (segment (start 114 90) (end 114 81.5) (width 0.5) (layer "B.Cu") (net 5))
 (segment (start 113.5 81) (end 112 81) (width 0.5) (layer "B.Cu") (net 5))
 (segment (start 129.08 93.905) (end 129.08 92.08) (width 0.5) (layer "B.Cu") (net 5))
 (segment (start 129.08 92.08) (end 128 91) (width 0.5) (layer "B.Cu") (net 5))
 (segment (start 153.15 75) (end 153.15 77.65) (width 0.5) (layer "B.Cu") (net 9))
 (segment (start 154.5 79) (end 154.5 81) (width 0.5) (layer "B.Cu") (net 9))
 (segment (start 154.5 79) (end 153.15 77.65) (width 0.5) (layer "B.Cu") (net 9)))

